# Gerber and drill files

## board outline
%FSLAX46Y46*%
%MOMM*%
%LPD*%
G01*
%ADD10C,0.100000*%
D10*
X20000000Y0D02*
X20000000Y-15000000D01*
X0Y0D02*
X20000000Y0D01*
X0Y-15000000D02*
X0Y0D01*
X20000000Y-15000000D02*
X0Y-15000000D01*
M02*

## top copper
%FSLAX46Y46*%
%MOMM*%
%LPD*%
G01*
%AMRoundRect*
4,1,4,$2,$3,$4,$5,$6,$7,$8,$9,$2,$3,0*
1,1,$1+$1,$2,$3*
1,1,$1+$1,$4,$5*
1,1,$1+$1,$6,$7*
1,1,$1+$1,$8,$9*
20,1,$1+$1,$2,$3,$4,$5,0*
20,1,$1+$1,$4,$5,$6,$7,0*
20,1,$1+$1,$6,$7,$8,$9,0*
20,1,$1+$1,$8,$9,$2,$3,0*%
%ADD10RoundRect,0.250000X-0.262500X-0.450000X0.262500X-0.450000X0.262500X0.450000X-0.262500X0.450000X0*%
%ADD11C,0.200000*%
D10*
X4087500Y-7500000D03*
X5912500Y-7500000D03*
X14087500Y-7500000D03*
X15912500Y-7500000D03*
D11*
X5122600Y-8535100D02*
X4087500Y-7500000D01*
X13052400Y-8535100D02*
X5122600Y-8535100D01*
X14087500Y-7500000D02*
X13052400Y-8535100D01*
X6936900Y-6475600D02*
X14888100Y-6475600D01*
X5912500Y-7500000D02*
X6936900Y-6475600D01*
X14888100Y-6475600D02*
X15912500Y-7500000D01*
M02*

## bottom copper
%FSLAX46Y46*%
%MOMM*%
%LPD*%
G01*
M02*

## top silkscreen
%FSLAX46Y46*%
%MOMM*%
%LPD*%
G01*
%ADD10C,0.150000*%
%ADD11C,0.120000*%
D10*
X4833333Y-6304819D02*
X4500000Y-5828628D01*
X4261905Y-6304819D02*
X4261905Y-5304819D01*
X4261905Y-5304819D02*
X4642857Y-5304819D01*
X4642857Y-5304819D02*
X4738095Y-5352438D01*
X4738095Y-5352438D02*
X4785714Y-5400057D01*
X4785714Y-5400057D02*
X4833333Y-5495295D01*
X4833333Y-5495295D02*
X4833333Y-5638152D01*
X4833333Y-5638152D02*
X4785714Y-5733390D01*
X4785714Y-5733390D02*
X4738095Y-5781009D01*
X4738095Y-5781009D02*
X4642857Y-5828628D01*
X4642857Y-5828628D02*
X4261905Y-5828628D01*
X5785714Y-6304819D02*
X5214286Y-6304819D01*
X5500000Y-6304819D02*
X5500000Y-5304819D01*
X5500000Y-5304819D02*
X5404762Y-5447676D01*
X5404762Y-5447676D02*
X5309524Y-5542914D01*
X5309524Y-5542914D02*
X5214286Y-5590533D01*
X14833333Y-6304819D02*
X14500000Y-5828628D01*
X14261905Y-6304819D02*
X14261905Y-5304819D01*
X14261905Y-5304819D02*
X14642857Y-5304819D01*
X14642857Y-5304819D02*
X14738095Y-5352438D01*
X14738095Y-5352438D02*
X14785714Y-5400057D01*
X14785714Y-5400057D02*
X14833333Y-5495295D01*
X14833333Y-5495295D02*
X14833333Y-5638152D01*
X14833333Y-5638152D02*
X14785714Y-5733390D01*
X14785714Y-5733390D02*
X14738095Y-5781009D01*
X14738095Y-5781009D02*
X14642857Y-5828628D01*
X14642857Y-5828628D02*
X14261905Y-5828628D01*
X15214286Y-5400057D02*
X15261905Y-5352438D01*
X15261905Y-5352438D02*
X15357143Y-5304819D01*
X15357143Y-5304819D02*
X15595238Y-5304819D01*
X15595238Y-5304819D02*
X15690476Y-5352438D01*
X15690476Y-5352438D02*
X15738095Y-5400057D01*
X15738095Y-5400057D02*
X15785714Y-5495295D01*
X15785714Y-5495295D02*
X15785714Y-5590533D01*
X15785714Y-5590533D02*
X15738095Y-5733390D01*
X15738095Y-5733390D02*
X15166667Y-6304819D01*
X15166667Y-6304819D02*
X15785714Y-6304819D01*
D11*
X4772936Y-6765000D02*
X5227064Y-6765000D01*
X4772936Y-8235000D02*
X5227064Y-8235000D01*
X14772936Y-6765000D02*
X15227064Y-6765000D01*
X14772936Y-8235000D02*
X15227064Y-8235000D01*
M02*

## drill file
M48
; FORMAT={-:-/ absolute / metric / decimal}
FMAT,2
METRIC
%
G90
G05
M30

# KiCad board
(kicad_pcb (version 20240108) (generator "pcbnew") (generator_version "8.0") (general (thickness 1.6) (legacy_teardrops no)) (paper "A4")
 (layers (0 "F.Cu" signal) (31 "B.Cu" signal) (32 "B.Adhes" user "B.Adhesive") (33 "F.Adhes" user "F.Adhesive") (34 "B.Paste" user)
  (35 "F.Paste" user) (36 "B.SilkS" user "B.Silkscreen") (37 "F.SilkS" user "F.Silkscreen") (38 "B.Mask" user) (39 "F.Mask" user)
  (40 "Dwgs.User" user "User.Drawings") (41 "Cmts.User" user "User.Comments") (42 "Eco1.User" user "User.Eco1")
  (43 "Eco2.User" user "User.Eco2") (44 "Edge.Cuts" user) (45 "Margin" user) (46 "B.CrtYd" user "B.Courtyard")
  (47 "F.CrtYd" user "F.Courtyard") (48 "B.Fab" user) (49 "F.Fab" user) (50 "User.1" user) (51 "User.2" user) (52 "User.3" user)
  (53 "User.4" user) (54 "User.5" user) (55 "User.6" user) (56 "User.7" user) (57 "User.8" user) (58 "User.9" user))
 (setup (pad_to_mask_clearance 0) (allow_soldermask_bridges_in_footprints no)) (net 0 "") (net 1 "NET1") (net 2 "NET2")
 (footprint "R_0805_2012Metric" (layer "F.Cu") (at 5 7.5)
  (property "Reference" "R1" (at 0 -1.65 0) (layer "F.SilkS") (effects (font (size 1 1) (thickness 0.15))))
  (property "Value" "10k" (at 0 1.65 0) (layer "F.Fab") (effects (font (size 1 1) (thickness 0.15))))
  (fp_line (start -0.227064 -0.735) (end 0.227064 -0.735) (stroke (width 0.12) (type solid)) (layer "F.SilkS"))
  (fp_line (start -0.227064 0.735) (end 0.227064 0.735) (stroke (width 0.12) (type solid)) (layer "F.SilkS"))
  (pad "1" smd roundrect (at -0.9125 0) (size 1.025 1.4) (layers "F.Cu" "F.Paste" "F.Mask") (roundrect_rratio 0.243902) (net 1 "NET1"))
  (pad "2" smd roundrect (at 0.9125 0) (size 1.025 1.4) (layers "F.Cu" "F.Paste" "F.Mask") (roundrect_rratio 0.243902) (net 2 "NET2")))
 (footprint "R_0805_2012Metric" (layer "F.Cu") (at 15 7.5)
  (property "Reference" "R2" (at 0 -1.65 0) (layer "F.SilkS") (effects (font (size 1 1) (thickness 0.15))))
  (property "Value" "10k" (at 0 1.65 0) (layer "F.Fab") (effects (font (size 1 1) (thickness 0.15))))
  (fp_line (start -0.227064 -0.735) (end 0.227064 -0.735) (stroke (width 0.12) (type solid)) (layer "F.SilkS"))
  (fp_line (start -0.227064 0.735) (end 0.227064 0.735) (stroke (width 0.12) (type solid)) (layer "F.SilkS"))
  (pad "1" smd roundrect (at -0.9125 0) (size 1.025 1.4) (layers "F.Cu" "F.Paste" "F.Mask") (roundrect_rratio 0.243902) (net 1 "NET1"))
  (pad "2" smd roundrect (at 0.9125 0) (size 1.025 1.4) (layers "F.Cu" "F.Paste" "F.Mask") (roundrect_rratio 0.243902) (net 2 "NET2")))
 (gr_line (start 20 0) (end 20 15) (stroke (width 0.1) (type default)) (layer "Edge.Cuts"))
 (gr_line (start 0 0) (end 20 0) (stroke (width 0.1) (type default)) (layer "Edge.Cuts"))
 (gr_line (start 0 15) (end 0 0) (stroke (width 0.1) (type default)) (layer "Edge.Cuts"))
 (gr_line (start 20 15) (end 0 15) (stroke (width 0.1) (type default)) (layer "Edge.Cuts"))
 (segment (start 5.1226 8.5351) (end 4.0875 7.5) (width 0.2) (layer "F.Cu") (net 1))
 (segment (start 13.0524 8.5351) (end 5.1226 8.5351) (width 0.2) (layer "F.Cu") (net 1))
 (segment (start 14.0875 7.5) (end 13.0524 8.5351) (width 0.2) (layer "F.Cu") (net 1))
 (segment (start 6.9369 6.4756) (end 14.8881 6.4756) (width 0.2) (layer "F.Cu") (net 2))
 (segment (start 5.9125 7.5) (end 6.9369 6.4756) (width 0.2) (layer "F.Cu") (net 2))
 (segment (start 14.8881 6.4756) (end 15.9125 7.5) (width 0.2) (layer "F.Cu") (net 2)))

